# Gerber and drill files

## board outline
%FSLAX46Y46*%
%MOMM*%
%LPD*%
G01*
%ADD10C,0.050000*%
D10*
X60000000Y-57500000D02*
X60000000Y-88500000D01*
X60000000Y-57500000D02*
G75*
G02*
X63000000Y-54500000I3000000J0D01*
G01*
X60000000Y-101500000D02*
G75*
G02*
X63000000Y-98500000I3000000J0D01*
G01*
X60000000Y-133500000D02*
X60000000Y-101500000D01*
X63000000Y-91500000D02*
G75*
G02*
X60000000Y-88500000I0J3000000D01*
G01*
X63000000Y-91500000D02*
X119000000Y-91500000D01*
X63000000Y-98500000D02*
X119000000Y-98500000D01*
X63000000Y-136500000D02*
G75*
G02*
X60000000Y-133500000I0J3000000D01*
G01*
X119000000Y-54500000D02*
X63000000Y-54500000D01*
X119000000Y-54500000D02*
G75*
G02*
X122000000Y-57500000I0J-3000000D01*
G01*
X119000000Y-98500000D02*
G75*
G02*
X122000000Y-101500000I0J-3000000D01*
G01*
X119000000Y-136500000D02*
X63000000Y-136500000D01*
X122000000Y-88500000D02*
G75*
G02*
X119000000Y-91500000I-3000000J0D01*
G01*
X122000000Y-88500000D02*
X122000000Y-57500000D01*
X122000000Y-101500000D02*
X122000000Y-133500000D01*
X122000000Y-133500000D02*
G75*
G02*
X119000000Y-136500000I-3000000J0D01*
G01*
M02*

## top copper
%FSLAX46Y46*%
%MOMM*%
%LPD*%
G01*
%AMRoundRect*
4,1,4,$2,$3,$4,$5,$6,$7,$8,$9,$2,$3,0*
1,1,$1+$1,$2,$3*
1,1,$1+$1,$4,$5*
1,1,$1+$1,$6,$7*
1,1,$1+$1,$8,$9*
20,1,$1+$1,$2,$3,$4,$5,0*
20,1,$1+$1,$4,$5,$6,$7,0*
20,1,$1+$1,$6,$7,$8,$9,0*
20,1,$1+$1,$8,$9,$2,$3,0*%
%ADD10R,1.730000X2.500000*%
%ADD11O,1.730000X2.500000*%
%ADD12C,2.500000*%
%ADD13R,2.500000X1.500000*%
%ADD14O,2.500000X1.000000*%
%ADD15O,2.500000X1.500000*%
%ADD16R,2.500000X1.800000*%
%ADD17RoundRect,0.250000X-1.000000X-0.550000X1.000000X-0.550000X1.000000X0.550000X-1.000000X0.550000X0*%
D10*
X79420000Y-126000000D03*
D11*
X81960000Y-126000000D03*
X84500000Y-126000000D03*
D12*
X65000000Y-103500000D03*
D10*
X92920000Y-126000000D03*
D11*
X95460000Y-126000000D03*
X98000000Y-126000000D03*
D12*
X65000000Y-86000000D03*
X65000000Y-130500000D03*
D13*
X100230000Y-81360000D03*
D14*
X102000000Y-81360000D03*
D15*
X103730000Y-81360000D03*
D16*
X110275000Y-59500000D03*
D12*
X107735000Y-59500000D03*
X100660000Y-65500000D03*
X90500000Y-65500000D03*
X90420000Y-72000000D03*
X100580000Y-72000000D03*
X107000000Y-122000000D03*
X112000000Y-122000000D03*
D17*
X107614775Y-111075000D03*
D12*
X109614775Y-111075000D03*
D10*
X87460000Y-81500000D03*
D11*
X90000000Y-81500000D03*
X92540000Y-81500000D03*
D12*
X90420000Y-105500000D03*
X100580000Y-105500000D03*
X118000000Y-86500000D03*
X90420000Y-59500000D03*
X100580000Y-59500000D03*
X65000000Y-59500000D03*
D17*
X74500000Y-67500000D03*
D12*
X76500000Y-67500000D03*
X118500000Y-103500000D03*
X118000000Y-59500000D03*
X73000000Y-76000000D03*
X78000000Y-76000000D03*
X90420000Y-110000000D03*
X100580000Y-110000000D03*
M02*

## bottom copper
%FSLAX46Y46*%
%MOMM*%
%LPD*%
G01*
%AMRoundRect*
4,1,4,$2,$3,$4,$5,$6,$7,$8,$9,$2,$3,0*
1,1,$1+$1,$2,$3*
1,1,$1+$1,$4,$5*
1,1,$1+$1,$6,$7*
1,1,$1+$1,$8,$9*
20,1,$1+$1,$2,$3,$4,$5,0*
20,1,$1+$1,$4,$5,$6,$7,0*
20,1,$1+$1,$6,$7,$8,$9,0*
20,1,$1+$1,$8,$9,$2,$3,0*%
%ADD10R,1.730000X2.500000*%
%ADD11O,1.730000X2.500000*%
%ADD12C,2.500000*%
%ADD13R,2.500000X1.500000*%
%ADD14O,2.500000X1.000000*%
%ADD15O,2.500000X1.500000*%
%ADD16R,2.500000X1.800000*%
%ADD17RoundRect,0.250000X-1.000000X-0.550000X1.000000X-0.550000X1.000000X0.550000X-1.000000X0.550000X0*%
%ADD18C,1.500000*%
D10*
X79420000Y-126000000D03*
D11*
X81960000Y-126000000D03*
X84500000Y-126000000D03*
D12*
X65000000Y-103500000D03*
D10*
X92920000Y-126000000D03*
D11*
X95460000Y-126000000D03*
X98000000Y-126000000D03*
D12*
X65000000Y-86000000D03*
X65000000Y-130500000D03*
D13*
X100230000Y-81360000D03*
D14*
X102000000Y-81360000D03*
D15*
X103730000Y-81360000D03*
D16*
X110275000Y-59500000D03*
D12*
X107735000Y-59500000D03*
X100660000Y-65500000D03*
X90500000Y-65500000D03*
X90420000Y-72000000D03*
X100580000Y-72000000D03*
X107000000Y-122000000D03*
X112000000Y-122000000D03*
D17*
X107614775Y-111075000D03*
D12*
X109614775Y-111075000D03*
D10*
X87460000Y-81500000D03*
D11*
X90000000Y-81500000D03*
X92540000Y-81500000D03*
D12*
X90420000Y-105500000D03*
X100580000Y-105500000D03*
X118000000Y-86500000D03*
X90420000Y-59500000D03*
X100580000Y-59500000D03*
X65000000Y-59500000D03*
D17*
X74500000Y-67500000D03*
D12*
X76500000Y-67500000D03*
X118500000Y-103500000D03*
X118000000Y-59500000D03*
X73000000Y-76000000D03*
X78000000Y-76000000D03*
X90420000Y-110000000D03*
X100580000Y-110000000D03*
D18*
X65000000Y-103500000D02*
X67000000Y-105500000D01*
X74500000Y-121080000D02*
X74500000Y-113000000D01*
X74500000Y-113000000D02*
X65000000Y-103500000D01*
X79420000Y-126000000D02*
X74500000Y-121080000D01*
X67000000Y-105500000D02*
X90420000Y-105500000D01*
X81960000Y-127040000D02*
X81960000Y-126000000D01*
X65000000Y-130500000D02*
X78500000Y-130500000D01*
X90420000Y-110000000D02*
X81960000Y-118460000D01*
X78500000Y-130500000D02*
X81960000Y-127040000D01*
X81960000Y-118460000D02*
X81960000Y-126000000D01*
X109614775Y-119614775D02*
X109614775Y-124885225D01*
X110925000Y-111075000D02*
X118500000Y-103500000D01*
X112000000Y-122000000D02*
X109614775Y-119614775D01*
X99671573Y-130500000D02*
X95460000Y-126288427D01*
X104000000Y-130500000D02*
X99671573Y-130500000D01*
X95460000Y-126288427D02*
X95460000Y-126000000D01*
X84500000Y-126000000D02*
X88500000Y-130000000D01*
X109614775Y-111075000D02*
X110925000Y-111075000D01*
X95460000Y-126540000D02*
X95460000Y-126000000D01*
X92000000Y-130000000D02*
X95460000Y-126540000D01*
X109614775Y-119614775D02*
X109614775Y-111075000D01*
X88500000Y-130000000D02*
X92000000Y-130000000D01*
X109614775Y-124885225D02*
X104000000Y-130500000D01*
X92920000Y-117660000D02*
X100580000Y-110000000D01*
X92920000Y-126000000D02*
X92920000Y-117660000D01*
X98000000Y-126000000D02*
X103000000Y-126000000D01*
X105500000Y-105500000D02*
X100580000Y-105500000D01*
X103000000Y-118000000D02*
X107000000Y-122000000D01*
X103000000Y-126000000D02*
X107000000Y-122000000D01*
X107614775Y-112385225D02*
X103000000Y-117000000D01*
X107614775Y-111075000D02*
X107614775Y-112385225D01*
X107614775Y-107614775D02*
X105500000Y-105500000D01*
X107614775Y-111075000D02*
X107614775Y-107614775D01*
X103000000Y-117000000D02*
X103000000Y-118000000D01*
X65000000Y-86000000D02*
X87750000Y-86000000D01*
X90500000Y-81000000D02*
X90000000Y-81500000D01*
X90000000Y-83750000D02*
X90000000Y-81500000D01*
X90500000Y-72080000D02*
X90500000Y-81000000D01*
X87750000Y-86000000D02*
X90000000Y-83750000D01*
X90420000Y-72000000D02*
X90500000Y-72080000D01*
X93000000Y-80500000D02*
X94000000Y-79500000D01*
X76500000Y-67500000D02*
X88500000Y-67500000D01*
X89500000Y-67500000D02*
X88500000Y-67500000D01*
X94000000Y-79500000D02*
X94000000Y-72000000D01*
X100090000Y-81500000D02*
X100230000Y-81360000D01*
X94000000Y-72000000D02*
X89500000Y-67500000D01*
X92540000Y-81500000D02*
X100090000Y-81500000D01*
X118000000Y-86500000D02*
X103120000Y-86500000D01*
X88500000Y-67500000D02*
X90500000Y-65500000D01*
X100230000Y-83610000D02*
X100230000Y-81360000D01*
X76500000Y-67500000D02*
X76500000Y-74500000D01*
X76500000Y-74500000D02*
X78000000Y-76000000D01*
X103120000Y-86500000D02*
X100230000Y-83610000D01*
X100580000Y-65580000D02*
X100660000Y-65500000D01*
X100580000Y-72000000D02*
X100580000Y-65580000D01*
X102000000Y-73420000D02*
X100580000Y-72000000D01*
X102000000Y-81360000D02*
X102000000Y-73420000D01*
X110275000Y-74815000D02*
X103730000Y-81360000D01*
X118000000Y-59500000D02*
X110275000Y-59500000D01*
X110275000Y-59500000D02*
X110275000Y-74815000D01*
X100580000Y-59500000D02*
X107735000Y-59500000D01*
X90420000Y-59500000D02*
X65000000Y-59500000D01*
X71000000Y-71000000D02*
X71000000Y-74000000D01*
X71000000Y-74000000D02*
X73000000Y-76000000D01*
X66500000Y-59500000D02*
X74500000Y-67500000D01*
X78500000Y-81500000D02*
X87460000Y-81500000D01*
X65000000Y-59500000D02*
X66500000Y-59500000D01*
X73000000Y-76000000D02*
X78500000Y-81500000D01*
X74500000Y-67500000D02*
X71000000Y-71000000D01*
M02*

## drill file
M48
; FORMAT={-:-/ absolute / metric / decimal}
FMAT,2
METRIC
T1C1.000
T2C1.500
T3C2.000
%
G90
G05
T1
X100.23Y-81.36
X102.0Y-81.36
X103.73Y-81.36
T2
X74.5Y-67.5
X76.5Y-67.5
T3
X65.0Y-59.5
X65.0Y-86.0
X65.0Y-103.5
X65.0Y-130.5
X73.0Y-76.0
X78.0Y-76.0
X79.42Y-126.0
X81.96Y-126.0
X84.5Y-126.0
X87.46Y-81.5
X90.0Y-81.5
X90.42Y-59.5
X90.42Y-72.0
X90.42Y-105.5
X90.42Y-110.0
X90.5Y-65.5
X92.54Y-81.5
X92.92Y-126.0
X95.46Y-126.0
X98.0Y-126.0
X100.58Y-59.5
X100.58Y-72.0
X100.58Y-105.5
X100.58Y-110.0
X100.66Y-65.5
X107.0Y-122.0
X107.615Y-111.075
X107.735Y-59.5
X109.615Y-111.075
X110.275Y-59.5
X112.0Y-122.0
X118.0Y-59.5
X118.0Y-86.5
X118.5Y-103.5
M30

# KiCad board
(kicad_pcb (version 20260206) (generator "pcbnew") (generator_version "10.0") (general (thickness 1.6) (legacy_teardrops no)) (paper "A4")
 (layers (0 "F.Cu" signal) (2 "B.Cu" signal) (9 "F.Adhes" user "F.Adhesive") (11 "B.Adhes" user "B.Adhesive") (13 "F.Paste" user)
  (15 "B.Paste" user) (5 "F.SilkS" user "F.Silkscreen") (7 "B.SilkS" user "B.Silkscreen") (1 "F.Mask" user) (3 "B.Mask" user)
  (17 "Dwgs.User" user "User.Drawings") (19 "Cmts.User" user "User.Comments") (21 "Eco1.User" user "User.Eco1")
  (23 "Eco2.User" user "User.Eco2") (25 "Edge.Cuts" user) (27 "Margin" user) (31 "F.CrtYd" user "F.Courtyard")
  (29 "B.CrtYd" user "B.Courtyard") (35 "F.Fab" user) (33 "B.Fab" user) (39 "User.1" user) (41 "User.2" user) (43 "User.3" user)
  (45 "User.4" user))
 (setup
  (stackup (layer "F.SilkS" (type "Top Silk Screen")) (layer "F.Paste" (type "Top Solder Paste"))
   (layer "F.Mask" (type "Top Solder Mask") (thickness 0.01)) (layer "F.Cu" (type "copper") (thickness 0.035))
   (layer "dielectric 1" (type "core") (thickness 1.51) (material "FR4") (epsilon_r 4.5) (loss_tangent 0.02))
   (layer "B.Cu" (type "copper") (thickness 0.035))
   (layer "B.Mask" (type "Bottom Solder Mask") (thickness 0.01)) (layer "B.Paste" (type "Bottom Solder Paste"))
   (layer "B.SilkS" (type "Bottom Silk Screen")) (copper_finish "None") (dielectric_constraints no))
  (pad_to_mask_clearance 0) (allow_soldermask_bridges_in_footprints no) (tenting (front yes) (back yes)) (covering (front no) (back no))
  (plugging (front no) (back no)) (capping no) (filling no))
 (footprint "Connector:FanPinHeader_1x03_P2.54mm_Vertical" (layer "F.Cu") (at 79.42 126)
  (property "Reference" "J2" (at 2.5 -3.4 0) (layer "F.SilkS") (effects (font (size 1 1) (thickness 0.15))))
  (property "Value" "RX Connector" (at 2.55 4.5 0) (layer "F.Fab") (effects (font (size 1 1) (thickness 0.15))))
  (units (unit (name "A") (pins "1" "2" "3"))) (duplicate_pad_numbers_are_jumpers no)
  (pad "1" thru_hole rect (at 0 0 90) (size 2.5 1.73) (drill 2) (layers "*.Cu" "*.Mask") (remove_unused_layers no) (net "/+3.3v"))
  (pad "2" thru_hole oval (at 2.54 0 90) (size 2.5 1.73) (drill 2) (layers "*.Cu" "*.Mask") (remove_unused_layers no) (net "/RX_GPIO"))
  (pad "3" thru_hole oval (at 5.08 0 90) (size 2.5 1.73) (drill 2) (layers "*.Cu" "*.Mask") (remove_unused_layers no) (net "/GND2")))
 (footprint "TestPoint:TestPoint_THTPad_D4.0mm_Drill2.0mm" (layer "F.Cu") (at 65 103.5)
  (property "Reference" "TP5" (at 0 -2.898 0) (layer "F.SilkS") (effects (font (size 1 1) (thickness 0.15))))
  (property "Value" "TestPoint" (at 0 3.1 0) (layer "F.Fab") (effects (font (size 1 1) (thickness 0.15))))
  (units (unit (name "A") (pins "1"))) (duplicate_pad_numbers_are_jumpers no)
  (pad "1" thru_hole circle (at 0 0) (size 2.5 2.5) (drill 2) (layers "*.Cu" "*.Mask") (remove_unused_layers no) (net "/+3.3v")))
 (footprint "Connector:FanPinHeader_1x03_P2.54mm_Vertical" (layer "F.Cu") (at 92.92 126)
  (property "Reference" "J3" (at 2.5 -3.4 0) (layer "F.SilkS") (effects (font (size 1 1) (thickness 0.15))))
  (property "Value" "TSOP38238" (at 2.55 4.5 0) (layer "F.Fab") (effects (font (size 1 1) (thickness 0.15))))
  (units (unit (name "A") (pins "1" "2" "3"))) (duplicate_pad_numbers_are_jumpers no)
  (pad "1" thru_hole rect (at 0 0 90) (size 2.5 1.73) (drill 2) (layers "*.Cu" "*.Mask") (remove_unused_layers no) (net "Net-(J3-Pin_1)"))
  (pad "2" thru_hole oval (at 2.54 0 90) (size 2.5 1.73) (drill 2) (layers "*.Cu" "*.Mask") (remove_unused_layers no) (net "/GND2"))
  (pad "3" thru_hole oval (at 5.08 0 90) (size 2.5 1.73) (drill 2) (layers "*.Cu" "*.Mask") (remove_unused_layers no)
   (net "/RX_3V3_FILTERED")))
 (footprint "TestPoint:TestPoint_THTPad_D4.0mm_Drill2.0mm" (layer "F.Cu") (at 65 86)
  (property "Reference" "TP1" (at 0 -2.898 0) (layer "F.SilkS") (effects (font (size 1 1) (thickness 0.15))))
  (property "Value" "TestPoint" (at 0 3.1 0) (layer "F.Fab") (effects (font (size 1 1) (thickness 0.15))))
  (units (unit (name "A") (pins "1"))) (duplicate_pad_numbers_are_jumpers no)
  (pad "1" thru_hole circle (at 0 0) (size 2.5 2.5) (drill 2) (layers "*.Cu" "*.Mask") (remove_unused_layers no) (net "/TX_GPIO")))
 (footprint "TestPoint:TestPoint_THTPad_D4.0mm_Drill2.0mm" (layer "F.Cu") (at 65 130.5)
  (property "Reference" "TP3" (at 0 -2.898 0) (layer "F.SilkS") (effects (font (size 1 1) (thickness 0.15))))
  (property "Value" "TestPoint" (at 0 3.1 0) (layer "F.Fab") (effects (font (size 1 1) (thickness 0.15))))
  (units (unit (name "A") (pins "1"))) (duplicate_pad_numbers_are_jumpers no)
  (pad "1" thru_hole circle (at 0 0) (size 2.5 2.5) (drill 2) (layers "*.Cu" "*.Mask") (remove_unused_layers no) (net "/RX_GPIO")))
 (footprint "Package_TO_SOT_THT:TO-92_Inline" (layer "F.Cu") (at 100.73 81.36)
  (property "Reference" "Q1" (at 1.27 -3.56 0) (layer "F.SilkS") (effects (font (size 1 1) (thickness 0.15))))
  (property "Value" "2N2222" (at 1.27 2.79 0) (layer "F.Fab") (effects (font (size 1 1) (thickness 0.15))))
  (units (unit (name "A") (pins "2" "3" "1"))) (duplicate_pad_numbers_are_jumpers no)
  (pad "1" thru_hole rect (at -0.5 0) (size 2.5 1.5) (drill 1) (layers "*.Cu" "*.Mask") (remove_unused_layers no) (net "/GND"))
  (pad "2" thru_hole oval (at 1.27 0) (size 2.5 1) (drill 1) (layers "*.Cu" "*.Mask") (remove_unused_layers no) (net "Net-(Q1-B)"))
  (pad "3" thru_hole oval (at 3 0) (size 2.5 1.5) (drill 1) (layers "*.Cu" "*.Mask") (remove_unused_layers no) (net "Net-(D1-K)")))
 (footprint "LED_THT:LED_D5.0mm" (layer "F.Cu") (at 110.275 59.5 180)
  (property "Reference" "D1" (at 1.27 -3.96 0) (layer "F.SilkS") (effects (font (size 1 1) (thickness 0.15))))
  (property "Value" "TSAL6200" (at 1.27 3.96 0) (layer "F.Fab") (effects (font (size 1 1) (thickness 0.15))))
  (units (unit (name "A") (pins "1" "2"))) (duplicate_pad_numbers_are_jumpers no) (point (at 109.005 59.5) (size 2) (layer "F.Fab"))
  (pad "1" thru_hole rect (at 0 0 180) (size 2.5 1.8) (drill 2) (layers "*.Cu" "*.Mask") (remove_unused_layers no) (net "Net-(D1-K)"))
  (pad "2" thru_hole circle (at 2.54 0 180) (size 2.5 2.5) (drill 2) (layers "*.Cu" "*.Mask") (remove_unused_layers no) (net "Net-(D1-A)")))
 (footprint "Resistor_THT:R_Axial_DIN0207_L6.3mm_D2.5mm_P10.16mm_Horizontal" (layer "F.Cu") (at 100.66 65.5 180)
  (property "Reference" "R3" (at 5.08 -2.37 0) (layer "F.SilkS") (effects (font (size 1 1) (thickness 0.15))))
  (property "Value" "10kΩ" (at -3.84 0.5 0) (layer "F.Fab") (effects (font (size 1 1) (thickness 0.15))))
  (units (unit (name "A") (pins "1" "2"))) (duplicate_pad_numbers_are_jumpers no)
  (pad "1" thru_hole circle (at 0 0 180) (size 2.5 2.5) (drill 2) (layers "*.Cu" "*.Mask") (remove_unused_layers no) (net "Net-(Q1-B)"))
  (pad "2" thru_hole circle (at 10.16 0 180) (size 2.5 2.5) (drill 2) (layers "*.Cu" "*.Mask") (remove_unused_layers no) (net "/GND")))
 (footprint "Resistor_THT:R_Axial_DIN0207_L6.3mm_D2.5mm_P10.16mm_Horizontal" (layer "F.Cu") (at 90.42 72)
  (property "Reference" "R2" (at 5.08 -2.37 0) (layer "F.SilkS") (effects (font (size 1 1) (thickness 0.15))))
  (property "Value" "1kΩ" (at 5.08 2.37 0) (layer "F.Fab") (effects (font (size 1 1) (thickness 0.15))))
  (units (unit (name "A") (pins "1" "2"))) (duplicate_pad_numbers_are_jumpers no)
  (pad "1" thru_hole circle (at 0 0) (size 2.5 2.5) (drill 2) (layers "*.Cu" "*.Mask") (remove_unused_layers no) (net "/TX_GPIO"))
  (pad "2" thru_hole circle (at 10.16 0) (size 2.5 2.5) (drill 2) (layers "*.Cu" "*.Mask") (remove_unused_layers no) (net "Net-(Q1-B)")))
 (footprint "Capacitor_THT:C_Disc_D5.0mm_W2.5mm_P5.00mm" (layer "F.Cu") (at 107 122)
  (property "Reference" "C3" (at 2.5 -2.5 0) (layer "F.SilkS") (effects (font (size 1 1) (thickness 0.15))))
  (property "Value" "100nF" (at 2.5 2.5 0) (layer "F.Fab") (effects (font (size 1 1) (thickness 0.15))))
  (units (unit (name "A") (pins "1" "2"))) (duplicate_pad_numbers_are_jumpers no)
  (pad "1" thru_hole circle (at 0 0) (size 2.5 2.5) (drill 2) (layers "*.Cu" "*.Mask") (remove_unused_layers no) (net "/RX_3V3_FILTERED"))
  (pad "2" thru_hole circle (at 5 0) (size 2.5 2.5) (drill 2) (layers "*.Cu" "*.Mask") (remove_unused_layers no) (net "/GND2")))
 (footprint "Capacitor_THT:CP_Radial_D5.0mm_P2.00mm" (layer "F.Cu") (at 107.614775 111.075)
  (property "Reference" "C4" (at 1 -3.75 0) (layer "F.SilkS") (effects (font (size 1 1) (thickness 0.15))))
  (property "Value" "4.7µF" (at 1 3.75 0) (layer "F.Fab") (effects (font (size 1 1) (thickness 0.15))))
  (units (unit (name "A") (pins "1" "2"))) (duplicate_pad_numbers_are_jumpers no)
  (pad "1" thru_hole roundrect (at 0 0) (size 2.5 1.6) (drill 2) (layers "*.Cu" "*.Mask") (remove_unused_layers no)
   (roundrect_rratio 0.15625) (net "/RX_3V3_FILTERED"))
  (pad "2" thru_hole circle (at 2 0) (size 2.5 2.5) (drill 2) (layers "*.Cu" "*.Mask") (remove_unused_layers no) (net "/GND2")))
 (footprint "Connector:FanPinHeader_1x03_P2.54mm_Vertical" (layer "F.Cu") (at 87.46 81.5)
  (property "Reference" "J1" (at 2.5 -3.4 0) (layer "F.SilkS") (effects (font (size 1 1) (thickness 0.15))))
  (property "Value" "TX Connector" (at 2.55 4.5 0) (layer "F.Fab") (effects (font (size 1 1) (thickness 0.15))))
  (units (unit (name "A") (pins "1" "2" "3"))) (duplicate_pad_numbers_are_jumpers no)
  (pad "1" thru_hole rect (at 0 0 90) (size 2.5 1.73) (drill 2) (layers "*.Cu" "*.Mask") (remove_unused_layers no) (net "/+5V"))
  (pad "2" thru_hole oval (at 2.54 0 90) (size 2.5 1.73) (drill 2) (layers "*.Cu" "*.Mask") (remove_unused_layers no) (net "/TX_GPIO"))
  (pad "3" thru_hole oval (at 5.08 0 90) (size 2.5 1.73) (drill 2) (layers "*.Cu" "*.Mask") (remove_unused_layers no) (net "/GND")))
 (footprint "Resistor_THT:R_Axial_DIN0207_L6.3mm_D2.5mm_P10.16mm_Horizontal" (layer "F.Cu") (at 90.42 105.5)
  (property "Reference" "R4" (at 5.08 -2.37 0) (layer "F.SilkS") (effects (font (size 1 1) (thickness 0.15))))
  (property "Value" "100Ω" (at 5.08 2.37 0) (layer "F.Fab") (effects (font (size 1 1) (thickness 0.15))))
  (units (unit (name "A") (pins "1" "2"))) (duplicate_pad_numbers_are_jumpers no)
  (pad "1" thru_hole circle (at 0 0) (size 2.5 2.5) (drill 2) (layers "*.Cu" "*.Mask") (remove_unused_layers no) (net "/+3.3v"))
  (pad "2" thru_hole circle (at 10.16 0) (size 2.5 2.5) (drill 2) (layers "*.Cu" "*.Mask") (remove_unused_layers no)
   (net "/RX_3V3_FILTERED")))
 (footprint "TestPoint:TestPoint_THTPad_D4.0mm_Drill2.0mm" (layer "F.Cu") (at 118 86.5)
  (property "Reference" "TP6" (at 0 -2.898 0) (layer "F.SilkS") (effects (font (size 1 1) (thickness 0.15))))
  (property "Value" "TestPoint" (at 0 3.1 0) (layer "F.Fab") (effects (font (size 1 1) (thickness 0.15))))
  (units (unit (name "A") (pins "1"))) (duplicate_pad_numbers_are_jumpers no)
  (pad "1" thru_hole circle (at 0 0) (size 2.5 2.5) (drill 2) (layers "*.Cu" "*.Mask") (remove_unused_layers no) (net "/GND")))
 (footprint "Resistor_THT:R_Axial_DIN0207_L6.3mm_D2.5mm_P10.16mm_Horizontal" (layer "F.Cu") (at 90.42 59.5)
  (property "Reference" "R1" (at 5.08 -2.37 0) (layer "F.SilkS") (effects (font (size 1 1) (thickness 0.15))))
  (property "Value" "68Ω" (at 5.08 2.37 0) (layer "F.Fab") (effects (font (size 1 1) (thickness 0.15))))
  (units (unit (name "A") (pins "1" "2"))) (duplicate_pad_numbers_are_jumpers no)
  (pad "1" thru_hole circle (at 0 0) (size 2.5 2.5) (drill 2) (layers "*.Cu" "*.Mask") (remove_unused_layers no) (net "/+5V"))
  (pad "2" thru_hole circle (at 10.16 0) (size 2.5 2.5) (drill 2) (layers "*.Cu" "*.Mask") (remove_unused_layers no) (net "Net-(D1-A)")))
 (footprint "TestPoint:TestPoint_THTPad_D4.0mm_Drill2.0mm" (layer "F.Cu") (at 65 59.5)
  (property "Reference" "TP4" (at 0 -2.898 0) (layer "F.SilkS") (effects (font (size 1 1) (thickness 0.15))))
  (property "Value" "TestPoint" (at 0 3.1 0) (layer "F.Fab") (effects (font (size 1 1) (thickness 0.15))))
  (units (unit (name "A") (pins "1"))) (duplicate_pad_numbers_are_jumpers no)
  (pad "1" thru_hole circle (at 0 0) (size 2.5 2.5) (drill 2) (layers "*.Cu" "*.Mask") (remove_unused_layers no) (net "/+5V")))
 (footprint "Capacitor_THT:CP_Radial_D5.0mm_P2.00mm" (layer "F.Cu") (at 74.5 67.5)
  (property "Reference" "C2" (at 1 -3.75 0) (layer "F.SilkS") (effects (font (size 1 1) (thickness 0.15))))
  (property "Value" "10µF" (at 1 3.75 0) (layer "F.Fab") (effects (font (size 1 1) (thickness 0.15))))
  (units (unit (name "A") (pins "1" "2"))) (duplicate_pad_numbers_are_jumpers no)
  (pad "1" thru_hole roundrect (at 0 0) (size 2.5 1.6) (drill 1.5) (layers "*.Cu" "*.Mask") (remove_unused_layers no)
   (roundrect_rratio 0.15625) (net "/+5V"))
  (pad "2" thru_hole circle (at 2 0) (size 2.5 2.5) (drill 1.5) (layers "*.Cu" "*.Mask") (remove_unused_layers no) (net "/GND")))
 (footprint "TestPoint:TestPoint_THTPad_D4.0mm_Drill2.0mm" (layer "F.Cu") (at 118.5 103.5)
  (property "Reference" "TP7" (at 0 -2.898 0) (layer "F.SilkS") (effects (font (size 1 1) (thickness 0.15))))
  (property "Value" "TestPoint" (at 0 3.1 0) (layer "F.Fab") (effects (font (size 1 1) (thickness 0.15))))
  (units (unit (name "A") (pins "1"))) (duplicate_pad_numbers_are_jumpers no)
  (pad "1" thru_hole circle (at 0 0) (size 2.5 2.5) (drill 2) (layers "*.Cu" "*.Mask") (remove_unused_layers no) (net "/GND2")))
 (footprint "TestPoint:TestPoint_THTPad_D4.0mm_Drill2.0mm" (layer "F.Cu") (at 118 59.5)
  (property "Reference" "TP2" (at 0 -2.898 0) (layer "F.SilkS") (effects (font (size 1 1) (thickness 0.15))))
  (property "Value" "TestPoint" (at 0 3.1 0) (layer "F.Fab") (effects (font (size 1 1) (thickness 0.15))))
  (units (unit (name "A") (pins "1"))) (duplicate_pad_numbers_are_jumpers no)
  (pad "1" thru_hole circle (at 0 0) (size 2.5 2.5) (drill 2) (layers "*.Cu" "*.Mask") (remove_unused_layers no) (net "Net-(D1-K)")))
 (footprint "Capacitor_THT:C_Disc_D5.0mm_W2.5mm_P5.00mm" (layer "F.Cu") (at 73 76)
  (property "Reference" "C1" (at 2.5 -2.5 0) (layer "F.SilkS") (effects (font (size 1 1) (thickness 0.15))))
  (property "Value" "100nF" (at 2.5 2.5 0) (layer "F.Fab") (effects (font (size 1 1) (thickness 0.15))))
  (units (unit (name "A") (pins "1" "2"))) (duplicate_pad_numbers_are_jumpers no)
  (pad "1" thru_hole circle (at 0 0) (size 2.5 2.5) (drill 2) (layers "*.Cu" "*.Mask") (remove_unused_layers no) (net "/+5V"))
  (pad "2" thru_hole circle (at 5 0) (size 2.5 2.5) (drill 2) (layers "*.Cu" "*.Mask") (remove_unused_layers no) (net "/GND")))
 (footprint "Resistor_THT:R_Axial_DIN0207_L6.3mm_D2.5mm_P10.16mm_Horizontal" (layer "F.Cu") (at 90.42 110)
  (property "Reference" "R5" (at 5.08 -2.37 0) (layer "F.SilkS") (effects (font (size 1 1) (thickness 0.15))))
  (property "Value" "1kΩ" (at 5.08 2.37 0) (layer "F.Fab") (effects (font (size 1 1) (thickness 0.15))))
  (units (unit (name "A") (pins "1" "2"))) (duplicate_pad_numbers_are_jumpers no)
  (pad "1" thru_hole circle (at 0 0) (size 2.5 2.5) (drill 2) (layers "*.Cu" "*.Mask") (remove_unused_layers no) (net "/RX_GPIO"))
  (pad "2" thru_hole circle (at 10.16 0) (size 2.5 2.5) (drill 2) (layers "*.Cu" "*.Mask") (remove_unused_layers no) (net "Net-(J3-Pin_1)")))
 (gr_line (start 60 57.5) (end 60 88.5) (stroke (width 0.05) (type default)) (layer "Edge.Cuts"))
 (gr_arc (start 60 57.5) (mid 60.87868 55.37868) (end 63 54.5) (stroke (width 0.05) (type default)) (layer "Edge.Cuts"))
 (gr_arc (start 60 101.5) (mid 60.87868 99.37868) (end 63 98.5) (stroke (width 0.05) (type default)) (layer "Edge.Cuts"))
 (gr_line (start 60 133.5) (end 60 101.5) (stroke (width 0.05) (type default)) (layer "Edge.Cuts"))
 (gr_arc (start 63 91.5) (mid 60.87868 90.62132) (end 60 88.5) (stroke (width 0.05) (type default)) (layer "Edge.Cuts"))
 (gr_line (start 63 91.5) (end 119 91.5) (stroke (width 0.05) (type default)) (layer "Edge.Cuts"))
 (gr_line (start 63 98.5) (end 119 98.5) (stroke (width 0.05) (type default)) (layer "Edge.Cuts"))
 (gr_arc (start 63 136.5) (mid 60.87868 135.62132) (end 60 133.5) (stroke (width 0.05) (type default)) (layer "Edge.Cuts"))
 (gr_line (start 119 54.5) (end 63 54.5) (stroke (width 0.05) (type default)) (layer "Edge.Cuts"))
 (gr_arc (start 119 54.5) (mid 121.12132 55.37868) (end 122 57.5) (stroke (width 0.05) (type default)) (layer "Edge.Cuts"))
 (gr_arc (start 119 98.5) (mid 121.12132 99.37868) (end 122 101.5) (stroke (width 0.05) (type default)) (layer "Edge.Cuts"))
 (gr_line (start 119 136.5) (end 63 136.5) (stroke (width 0.05) (type default)) (layer "Edge.Cuts"))
 (gr_arc (start 122 88.5) (mid 121.12132 90.62132) (end 119 91.5) (stroke (width 0.05) (type default)) (layer "Edge.Cuts"))
 (gr_line (start 122 88.5) (end 122 57.5) (stroke (width 0.05) (type default)) (layer "Edge.Cuts"))
 (gr_line (start 122 101.5) (end 122 133.5) (stroke (width 0.05) (type default)) (layer "Edge.Cuts"))
 (gr_arc (start 122 133.5) (mid 121.12132 135.62132) (end 119 136.5) (stroke (width 0.05) (type default)) (layer "Edge.Cuts"))
 (segment (start 65 103.5) (end 67 105.5) (width 1.5) (layer "B.Cu") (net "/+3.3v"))
 (segment (start 74.5 121.08) (end 74.5 113) (width 1.5) (layer "B.Cu") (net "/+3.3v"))
 (segment (start 74.5 113) (end 65 103.5) (width 1.5) (layer "B.Cu") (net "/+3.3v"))
 (segment (start 79.42 126) (end 74.5 121.08) (width 1.5) (layer "B.Cu") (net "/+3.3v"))
 (segment (start 67 105.5) (end 90.42 105.5) (width 1.5) (layer "B.Cu") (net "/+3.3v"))
 (segment (start 81.96 127.04) (end 81.96 126) (width 1.5) (layer "B.Cu") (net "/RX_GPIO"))
 (segment (start 65 130.5) (end 78.5 130.5) (width 1.5) (layer "B.Cu") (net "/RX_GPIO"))
 (segment (start 90.42 110) (end 81.96 118.46) (width 1.5) (layer "B.Cu") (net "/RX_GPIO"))
 (segment (start 78.5 130.5) (end 81.96 127.04) (width 1.5) (layer "B.Cu") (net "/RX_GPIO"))
 (segment (start 81.96 118.46) (end 81.96 126) (width 1.5) (layer "B.Cu") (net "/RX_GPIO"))
 (segment (start 109.614775 119.614775) (end 109.614775 124.885225) (width 1.5) (layer "B.Cu") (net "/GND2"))
 (segment (start 110.925 111.075) (end 118.5 103.5) (width 1.5) (layer "B.Cu") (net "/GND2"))
 (segment (start 112 122) (end 109.614775 119.614775) (width 1.5) (layer "B.Cu") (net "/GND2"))
 (segment (start 99.671573 130.5) (end 95.46 126.288427) (width 1.5) (layer "B.Cu") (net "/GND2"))
 (segment (start 104 130.5) (end 99.671573 130.5) (width 1.5) (layer "B.Cu") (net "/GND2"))
 (segment (start 95.46 126.288427) (end 95.46 126) (width 1.5) (layer "B.Cu") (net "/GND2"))
 (segment (start 84.5 126) (end 88.5 130) (width 1.5) (layer "B.Cu") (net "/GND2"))
 (segment (start 109.614775 111.075) (end 110.925 111.075) (width 1.5) (layer "B.Cu") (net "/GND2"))
 (segment (start 95.46 126.54) (end 95.46 126) (width 1.5) (layer "B.Cu") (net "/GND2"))
 (segment (start 92 130) (end 95.46 126.54) (width 1.5) (layer "B.Cu") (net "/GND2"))
 (segment (start 109.614775 119.614775) (end 109.614775 111.075) (width 1.5) (layer "B.Cu") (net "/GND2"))
 (segment (start 88.5 130) (end 92 130) (width 1.5) (layer "B.Cu") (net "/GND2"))
 (segment (start 109.614775 124.885225) (end 104 130.5) (width 1.5) (layer "B.Cu") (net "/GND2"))
 (segment (start 92.92 117.66) (end 100.58 110) (width 1.5) (layer "B.Cu") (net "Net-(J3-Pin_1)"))
 (segment (start 92.92 126) (end 92.92 117.66) (width 1.5) (layer "B.Cu") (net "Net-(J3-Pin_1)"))
 (segment (start 98 126) (end 103 126) (width 1.5) (layer "B.Cu") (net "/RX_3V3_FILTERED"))
 (segment (start 105.5 105.5) (end 100.58 105.5) (width 1.5) (layer "B.Cu") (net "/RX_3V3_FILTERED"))
 (segment (start 103 118) (end 107 122) (width 1.5) (layer "B.Cu") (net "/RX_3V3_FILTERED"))
 (segment (start 103 126) (end 107 122) (width 1.5) (layer "B.Cu") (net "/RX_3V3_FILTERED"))
 (segment (start 107.614775 112.385225) (end 103 117) (width 1.5) (layer "B.Cu") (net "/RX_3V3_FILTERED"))
 (segment (start 107.614775 111.075) (end 107.614775 112.385225) (width 1.5) (layer "B.Cu") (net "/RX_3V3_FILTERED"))
 (segment (start 107.614775 107.614775) (end 105.5 105.5) (width 1.5) (layer "B.Cu") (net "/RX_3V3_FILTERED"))
 (segment (start 107.614775 111.075) (end 107.614775 107.614775) (width 1.5) (layer "B.Cu") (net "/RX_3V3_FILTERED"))
 (segment (start 103 117) (end 103 118) (width 1.5) (layer "B.Cu") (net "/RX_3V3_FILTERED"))
 (segment (start 65 86) (end 87.75 86) (width 1.5) (layer "B.Cu") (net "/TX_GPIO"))
 (segment (start 90.5 81) (end 90 81.5) (width 1.5) (layer "B.Cu") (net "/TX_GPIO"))
 (segment (start 90 83.75) (end 90 81.5) (width 1.5) (layer "B.Cu") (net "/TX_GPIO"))
 (segment (start 90.5 72.08) (end 90.5 81) (width 1.5) (layer "B.Cu") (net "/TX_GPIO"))
 (segment (start 87.75 86) (end 90 83.75) (width 1.5) (layer "B.Cu") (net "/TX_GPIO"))
 (segment (start 90.42 72) (end 90.5 72.08) (width 1.5) (layer "B.Cu") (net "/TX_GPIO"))
 (segment (start 93 80.5) (end 94 79.5) (width 1.5) (layer "B.Cu") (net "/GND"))
 (segment (start 76.5 67.5) (end 88.5 67.5) (width 1.5) (layer "B.Cu") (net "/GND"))
 (segment (start 89.5 67.5) (end 88.5 67.5) (width 1.5) (layer "B.Cu") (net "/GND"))
 (segment (start 94 79.5) (end 94 72) (width 1.5) (layer "B.Cu") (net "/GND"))
 (segment (start 100.09 81.5) (end 100.23 81.36) (width 1.5) (layer "B.Cu") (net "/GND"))
 (segment (start 94 72) (end 89.5 67.5) (width 1.5) (layer "B.Cu") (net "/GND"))
 (segment (start 92.54 81.5) (end 100.09 81.5) (width 1.5) (layer "B.Cu") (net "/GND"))
 (segment (start 118 86.5) (end 103.12 86.5) (width 1.5) (layer "B.Cu") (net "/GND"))
 (segment (start 88.5 67.5) (end 90.5 65.5) (width 1.5) (layer "B.Cu") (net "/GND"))
 (segment (start 100.23 83.61) (end 100.23 81.36) (width 1.5) (layer "B.Cu") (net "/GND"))
 (segment (start 76.5 67.5) (end 76.5 74.5) (width 1.5) (layer "B.Cu") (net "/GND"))
 (segment (start 76.5 74.5) (end 78 76) (width 1.5) (layer "B.Cu") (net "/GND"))
 (segment (start 103.12 86.5) (end 100.23 83.61) (width 1.5) (layer "B.Cu") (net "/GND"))
 (segment (start 100.58 65.58) (end 100.66 65.5) (width 1.5) (layer "B.Cu") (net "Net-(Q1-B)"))
 (segment (start 100.58 72) (end 100.58 65.58) (width 1.5) (layer "B.Cu") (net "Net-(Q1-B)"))
 (segment (start 102 73.42) (end 100.58 72) (width 1.5) (layer "B.Cu") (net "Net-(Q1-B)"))
 (segment (start 102 81.36) (end 102 73.42) (width 1.5) (layer "B.Cu") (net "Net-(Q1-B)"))
 (segment (start 110.275 74.815) (end 103.73 81.36) (width 1.5) (layer "B.Cu") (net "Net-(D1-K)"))
 (segment (start 118 59.5) (end 110.275 59.5) (width 1.5) (layer "B.Cu") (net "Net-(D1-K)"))
 (segment (start 110.275 59.5) (end 110.275 74.815) (width 1.5) (layer "B.Cu") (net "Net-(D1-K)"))
 (segment (start 100.58 59.5) (end 107.735 59.5) (width 1.5) (layer "B.Cu") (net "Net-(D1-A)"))
 (segment (start 90.42 59.5) (end 65 59.5) (width 1.5) (layer "B.Cu") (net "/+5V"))
 (segment (start 71 71) (end 71 74) (width 1.5) (layer "B.Cu") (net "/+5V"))
 (segment (start 71 74) (end 73 76) (width 1.5) (layer "B.Cu") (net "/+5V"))
 (segment (start 66.5 59.5) (end 74.5 67.5) (width 1.5) (layer "B.Cu") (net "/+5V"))
 (segment (start 78.5 81.5) (end 87.46 81.5) (width 1.5) (layer "B.Cu") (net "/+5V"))
 (segment (start 65 59.5) (end 66.5 59.5) (width 1.5) (layer "B.Cu") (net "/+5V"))
 (segment (start 73 76) (end 78.5 81.5) (width 1.5) (layer "B.Cu") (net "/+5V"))
 (segment (start 74.5 67.5) (end 71 71) (width 1.5) (layer "B.Cu") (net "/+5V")))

